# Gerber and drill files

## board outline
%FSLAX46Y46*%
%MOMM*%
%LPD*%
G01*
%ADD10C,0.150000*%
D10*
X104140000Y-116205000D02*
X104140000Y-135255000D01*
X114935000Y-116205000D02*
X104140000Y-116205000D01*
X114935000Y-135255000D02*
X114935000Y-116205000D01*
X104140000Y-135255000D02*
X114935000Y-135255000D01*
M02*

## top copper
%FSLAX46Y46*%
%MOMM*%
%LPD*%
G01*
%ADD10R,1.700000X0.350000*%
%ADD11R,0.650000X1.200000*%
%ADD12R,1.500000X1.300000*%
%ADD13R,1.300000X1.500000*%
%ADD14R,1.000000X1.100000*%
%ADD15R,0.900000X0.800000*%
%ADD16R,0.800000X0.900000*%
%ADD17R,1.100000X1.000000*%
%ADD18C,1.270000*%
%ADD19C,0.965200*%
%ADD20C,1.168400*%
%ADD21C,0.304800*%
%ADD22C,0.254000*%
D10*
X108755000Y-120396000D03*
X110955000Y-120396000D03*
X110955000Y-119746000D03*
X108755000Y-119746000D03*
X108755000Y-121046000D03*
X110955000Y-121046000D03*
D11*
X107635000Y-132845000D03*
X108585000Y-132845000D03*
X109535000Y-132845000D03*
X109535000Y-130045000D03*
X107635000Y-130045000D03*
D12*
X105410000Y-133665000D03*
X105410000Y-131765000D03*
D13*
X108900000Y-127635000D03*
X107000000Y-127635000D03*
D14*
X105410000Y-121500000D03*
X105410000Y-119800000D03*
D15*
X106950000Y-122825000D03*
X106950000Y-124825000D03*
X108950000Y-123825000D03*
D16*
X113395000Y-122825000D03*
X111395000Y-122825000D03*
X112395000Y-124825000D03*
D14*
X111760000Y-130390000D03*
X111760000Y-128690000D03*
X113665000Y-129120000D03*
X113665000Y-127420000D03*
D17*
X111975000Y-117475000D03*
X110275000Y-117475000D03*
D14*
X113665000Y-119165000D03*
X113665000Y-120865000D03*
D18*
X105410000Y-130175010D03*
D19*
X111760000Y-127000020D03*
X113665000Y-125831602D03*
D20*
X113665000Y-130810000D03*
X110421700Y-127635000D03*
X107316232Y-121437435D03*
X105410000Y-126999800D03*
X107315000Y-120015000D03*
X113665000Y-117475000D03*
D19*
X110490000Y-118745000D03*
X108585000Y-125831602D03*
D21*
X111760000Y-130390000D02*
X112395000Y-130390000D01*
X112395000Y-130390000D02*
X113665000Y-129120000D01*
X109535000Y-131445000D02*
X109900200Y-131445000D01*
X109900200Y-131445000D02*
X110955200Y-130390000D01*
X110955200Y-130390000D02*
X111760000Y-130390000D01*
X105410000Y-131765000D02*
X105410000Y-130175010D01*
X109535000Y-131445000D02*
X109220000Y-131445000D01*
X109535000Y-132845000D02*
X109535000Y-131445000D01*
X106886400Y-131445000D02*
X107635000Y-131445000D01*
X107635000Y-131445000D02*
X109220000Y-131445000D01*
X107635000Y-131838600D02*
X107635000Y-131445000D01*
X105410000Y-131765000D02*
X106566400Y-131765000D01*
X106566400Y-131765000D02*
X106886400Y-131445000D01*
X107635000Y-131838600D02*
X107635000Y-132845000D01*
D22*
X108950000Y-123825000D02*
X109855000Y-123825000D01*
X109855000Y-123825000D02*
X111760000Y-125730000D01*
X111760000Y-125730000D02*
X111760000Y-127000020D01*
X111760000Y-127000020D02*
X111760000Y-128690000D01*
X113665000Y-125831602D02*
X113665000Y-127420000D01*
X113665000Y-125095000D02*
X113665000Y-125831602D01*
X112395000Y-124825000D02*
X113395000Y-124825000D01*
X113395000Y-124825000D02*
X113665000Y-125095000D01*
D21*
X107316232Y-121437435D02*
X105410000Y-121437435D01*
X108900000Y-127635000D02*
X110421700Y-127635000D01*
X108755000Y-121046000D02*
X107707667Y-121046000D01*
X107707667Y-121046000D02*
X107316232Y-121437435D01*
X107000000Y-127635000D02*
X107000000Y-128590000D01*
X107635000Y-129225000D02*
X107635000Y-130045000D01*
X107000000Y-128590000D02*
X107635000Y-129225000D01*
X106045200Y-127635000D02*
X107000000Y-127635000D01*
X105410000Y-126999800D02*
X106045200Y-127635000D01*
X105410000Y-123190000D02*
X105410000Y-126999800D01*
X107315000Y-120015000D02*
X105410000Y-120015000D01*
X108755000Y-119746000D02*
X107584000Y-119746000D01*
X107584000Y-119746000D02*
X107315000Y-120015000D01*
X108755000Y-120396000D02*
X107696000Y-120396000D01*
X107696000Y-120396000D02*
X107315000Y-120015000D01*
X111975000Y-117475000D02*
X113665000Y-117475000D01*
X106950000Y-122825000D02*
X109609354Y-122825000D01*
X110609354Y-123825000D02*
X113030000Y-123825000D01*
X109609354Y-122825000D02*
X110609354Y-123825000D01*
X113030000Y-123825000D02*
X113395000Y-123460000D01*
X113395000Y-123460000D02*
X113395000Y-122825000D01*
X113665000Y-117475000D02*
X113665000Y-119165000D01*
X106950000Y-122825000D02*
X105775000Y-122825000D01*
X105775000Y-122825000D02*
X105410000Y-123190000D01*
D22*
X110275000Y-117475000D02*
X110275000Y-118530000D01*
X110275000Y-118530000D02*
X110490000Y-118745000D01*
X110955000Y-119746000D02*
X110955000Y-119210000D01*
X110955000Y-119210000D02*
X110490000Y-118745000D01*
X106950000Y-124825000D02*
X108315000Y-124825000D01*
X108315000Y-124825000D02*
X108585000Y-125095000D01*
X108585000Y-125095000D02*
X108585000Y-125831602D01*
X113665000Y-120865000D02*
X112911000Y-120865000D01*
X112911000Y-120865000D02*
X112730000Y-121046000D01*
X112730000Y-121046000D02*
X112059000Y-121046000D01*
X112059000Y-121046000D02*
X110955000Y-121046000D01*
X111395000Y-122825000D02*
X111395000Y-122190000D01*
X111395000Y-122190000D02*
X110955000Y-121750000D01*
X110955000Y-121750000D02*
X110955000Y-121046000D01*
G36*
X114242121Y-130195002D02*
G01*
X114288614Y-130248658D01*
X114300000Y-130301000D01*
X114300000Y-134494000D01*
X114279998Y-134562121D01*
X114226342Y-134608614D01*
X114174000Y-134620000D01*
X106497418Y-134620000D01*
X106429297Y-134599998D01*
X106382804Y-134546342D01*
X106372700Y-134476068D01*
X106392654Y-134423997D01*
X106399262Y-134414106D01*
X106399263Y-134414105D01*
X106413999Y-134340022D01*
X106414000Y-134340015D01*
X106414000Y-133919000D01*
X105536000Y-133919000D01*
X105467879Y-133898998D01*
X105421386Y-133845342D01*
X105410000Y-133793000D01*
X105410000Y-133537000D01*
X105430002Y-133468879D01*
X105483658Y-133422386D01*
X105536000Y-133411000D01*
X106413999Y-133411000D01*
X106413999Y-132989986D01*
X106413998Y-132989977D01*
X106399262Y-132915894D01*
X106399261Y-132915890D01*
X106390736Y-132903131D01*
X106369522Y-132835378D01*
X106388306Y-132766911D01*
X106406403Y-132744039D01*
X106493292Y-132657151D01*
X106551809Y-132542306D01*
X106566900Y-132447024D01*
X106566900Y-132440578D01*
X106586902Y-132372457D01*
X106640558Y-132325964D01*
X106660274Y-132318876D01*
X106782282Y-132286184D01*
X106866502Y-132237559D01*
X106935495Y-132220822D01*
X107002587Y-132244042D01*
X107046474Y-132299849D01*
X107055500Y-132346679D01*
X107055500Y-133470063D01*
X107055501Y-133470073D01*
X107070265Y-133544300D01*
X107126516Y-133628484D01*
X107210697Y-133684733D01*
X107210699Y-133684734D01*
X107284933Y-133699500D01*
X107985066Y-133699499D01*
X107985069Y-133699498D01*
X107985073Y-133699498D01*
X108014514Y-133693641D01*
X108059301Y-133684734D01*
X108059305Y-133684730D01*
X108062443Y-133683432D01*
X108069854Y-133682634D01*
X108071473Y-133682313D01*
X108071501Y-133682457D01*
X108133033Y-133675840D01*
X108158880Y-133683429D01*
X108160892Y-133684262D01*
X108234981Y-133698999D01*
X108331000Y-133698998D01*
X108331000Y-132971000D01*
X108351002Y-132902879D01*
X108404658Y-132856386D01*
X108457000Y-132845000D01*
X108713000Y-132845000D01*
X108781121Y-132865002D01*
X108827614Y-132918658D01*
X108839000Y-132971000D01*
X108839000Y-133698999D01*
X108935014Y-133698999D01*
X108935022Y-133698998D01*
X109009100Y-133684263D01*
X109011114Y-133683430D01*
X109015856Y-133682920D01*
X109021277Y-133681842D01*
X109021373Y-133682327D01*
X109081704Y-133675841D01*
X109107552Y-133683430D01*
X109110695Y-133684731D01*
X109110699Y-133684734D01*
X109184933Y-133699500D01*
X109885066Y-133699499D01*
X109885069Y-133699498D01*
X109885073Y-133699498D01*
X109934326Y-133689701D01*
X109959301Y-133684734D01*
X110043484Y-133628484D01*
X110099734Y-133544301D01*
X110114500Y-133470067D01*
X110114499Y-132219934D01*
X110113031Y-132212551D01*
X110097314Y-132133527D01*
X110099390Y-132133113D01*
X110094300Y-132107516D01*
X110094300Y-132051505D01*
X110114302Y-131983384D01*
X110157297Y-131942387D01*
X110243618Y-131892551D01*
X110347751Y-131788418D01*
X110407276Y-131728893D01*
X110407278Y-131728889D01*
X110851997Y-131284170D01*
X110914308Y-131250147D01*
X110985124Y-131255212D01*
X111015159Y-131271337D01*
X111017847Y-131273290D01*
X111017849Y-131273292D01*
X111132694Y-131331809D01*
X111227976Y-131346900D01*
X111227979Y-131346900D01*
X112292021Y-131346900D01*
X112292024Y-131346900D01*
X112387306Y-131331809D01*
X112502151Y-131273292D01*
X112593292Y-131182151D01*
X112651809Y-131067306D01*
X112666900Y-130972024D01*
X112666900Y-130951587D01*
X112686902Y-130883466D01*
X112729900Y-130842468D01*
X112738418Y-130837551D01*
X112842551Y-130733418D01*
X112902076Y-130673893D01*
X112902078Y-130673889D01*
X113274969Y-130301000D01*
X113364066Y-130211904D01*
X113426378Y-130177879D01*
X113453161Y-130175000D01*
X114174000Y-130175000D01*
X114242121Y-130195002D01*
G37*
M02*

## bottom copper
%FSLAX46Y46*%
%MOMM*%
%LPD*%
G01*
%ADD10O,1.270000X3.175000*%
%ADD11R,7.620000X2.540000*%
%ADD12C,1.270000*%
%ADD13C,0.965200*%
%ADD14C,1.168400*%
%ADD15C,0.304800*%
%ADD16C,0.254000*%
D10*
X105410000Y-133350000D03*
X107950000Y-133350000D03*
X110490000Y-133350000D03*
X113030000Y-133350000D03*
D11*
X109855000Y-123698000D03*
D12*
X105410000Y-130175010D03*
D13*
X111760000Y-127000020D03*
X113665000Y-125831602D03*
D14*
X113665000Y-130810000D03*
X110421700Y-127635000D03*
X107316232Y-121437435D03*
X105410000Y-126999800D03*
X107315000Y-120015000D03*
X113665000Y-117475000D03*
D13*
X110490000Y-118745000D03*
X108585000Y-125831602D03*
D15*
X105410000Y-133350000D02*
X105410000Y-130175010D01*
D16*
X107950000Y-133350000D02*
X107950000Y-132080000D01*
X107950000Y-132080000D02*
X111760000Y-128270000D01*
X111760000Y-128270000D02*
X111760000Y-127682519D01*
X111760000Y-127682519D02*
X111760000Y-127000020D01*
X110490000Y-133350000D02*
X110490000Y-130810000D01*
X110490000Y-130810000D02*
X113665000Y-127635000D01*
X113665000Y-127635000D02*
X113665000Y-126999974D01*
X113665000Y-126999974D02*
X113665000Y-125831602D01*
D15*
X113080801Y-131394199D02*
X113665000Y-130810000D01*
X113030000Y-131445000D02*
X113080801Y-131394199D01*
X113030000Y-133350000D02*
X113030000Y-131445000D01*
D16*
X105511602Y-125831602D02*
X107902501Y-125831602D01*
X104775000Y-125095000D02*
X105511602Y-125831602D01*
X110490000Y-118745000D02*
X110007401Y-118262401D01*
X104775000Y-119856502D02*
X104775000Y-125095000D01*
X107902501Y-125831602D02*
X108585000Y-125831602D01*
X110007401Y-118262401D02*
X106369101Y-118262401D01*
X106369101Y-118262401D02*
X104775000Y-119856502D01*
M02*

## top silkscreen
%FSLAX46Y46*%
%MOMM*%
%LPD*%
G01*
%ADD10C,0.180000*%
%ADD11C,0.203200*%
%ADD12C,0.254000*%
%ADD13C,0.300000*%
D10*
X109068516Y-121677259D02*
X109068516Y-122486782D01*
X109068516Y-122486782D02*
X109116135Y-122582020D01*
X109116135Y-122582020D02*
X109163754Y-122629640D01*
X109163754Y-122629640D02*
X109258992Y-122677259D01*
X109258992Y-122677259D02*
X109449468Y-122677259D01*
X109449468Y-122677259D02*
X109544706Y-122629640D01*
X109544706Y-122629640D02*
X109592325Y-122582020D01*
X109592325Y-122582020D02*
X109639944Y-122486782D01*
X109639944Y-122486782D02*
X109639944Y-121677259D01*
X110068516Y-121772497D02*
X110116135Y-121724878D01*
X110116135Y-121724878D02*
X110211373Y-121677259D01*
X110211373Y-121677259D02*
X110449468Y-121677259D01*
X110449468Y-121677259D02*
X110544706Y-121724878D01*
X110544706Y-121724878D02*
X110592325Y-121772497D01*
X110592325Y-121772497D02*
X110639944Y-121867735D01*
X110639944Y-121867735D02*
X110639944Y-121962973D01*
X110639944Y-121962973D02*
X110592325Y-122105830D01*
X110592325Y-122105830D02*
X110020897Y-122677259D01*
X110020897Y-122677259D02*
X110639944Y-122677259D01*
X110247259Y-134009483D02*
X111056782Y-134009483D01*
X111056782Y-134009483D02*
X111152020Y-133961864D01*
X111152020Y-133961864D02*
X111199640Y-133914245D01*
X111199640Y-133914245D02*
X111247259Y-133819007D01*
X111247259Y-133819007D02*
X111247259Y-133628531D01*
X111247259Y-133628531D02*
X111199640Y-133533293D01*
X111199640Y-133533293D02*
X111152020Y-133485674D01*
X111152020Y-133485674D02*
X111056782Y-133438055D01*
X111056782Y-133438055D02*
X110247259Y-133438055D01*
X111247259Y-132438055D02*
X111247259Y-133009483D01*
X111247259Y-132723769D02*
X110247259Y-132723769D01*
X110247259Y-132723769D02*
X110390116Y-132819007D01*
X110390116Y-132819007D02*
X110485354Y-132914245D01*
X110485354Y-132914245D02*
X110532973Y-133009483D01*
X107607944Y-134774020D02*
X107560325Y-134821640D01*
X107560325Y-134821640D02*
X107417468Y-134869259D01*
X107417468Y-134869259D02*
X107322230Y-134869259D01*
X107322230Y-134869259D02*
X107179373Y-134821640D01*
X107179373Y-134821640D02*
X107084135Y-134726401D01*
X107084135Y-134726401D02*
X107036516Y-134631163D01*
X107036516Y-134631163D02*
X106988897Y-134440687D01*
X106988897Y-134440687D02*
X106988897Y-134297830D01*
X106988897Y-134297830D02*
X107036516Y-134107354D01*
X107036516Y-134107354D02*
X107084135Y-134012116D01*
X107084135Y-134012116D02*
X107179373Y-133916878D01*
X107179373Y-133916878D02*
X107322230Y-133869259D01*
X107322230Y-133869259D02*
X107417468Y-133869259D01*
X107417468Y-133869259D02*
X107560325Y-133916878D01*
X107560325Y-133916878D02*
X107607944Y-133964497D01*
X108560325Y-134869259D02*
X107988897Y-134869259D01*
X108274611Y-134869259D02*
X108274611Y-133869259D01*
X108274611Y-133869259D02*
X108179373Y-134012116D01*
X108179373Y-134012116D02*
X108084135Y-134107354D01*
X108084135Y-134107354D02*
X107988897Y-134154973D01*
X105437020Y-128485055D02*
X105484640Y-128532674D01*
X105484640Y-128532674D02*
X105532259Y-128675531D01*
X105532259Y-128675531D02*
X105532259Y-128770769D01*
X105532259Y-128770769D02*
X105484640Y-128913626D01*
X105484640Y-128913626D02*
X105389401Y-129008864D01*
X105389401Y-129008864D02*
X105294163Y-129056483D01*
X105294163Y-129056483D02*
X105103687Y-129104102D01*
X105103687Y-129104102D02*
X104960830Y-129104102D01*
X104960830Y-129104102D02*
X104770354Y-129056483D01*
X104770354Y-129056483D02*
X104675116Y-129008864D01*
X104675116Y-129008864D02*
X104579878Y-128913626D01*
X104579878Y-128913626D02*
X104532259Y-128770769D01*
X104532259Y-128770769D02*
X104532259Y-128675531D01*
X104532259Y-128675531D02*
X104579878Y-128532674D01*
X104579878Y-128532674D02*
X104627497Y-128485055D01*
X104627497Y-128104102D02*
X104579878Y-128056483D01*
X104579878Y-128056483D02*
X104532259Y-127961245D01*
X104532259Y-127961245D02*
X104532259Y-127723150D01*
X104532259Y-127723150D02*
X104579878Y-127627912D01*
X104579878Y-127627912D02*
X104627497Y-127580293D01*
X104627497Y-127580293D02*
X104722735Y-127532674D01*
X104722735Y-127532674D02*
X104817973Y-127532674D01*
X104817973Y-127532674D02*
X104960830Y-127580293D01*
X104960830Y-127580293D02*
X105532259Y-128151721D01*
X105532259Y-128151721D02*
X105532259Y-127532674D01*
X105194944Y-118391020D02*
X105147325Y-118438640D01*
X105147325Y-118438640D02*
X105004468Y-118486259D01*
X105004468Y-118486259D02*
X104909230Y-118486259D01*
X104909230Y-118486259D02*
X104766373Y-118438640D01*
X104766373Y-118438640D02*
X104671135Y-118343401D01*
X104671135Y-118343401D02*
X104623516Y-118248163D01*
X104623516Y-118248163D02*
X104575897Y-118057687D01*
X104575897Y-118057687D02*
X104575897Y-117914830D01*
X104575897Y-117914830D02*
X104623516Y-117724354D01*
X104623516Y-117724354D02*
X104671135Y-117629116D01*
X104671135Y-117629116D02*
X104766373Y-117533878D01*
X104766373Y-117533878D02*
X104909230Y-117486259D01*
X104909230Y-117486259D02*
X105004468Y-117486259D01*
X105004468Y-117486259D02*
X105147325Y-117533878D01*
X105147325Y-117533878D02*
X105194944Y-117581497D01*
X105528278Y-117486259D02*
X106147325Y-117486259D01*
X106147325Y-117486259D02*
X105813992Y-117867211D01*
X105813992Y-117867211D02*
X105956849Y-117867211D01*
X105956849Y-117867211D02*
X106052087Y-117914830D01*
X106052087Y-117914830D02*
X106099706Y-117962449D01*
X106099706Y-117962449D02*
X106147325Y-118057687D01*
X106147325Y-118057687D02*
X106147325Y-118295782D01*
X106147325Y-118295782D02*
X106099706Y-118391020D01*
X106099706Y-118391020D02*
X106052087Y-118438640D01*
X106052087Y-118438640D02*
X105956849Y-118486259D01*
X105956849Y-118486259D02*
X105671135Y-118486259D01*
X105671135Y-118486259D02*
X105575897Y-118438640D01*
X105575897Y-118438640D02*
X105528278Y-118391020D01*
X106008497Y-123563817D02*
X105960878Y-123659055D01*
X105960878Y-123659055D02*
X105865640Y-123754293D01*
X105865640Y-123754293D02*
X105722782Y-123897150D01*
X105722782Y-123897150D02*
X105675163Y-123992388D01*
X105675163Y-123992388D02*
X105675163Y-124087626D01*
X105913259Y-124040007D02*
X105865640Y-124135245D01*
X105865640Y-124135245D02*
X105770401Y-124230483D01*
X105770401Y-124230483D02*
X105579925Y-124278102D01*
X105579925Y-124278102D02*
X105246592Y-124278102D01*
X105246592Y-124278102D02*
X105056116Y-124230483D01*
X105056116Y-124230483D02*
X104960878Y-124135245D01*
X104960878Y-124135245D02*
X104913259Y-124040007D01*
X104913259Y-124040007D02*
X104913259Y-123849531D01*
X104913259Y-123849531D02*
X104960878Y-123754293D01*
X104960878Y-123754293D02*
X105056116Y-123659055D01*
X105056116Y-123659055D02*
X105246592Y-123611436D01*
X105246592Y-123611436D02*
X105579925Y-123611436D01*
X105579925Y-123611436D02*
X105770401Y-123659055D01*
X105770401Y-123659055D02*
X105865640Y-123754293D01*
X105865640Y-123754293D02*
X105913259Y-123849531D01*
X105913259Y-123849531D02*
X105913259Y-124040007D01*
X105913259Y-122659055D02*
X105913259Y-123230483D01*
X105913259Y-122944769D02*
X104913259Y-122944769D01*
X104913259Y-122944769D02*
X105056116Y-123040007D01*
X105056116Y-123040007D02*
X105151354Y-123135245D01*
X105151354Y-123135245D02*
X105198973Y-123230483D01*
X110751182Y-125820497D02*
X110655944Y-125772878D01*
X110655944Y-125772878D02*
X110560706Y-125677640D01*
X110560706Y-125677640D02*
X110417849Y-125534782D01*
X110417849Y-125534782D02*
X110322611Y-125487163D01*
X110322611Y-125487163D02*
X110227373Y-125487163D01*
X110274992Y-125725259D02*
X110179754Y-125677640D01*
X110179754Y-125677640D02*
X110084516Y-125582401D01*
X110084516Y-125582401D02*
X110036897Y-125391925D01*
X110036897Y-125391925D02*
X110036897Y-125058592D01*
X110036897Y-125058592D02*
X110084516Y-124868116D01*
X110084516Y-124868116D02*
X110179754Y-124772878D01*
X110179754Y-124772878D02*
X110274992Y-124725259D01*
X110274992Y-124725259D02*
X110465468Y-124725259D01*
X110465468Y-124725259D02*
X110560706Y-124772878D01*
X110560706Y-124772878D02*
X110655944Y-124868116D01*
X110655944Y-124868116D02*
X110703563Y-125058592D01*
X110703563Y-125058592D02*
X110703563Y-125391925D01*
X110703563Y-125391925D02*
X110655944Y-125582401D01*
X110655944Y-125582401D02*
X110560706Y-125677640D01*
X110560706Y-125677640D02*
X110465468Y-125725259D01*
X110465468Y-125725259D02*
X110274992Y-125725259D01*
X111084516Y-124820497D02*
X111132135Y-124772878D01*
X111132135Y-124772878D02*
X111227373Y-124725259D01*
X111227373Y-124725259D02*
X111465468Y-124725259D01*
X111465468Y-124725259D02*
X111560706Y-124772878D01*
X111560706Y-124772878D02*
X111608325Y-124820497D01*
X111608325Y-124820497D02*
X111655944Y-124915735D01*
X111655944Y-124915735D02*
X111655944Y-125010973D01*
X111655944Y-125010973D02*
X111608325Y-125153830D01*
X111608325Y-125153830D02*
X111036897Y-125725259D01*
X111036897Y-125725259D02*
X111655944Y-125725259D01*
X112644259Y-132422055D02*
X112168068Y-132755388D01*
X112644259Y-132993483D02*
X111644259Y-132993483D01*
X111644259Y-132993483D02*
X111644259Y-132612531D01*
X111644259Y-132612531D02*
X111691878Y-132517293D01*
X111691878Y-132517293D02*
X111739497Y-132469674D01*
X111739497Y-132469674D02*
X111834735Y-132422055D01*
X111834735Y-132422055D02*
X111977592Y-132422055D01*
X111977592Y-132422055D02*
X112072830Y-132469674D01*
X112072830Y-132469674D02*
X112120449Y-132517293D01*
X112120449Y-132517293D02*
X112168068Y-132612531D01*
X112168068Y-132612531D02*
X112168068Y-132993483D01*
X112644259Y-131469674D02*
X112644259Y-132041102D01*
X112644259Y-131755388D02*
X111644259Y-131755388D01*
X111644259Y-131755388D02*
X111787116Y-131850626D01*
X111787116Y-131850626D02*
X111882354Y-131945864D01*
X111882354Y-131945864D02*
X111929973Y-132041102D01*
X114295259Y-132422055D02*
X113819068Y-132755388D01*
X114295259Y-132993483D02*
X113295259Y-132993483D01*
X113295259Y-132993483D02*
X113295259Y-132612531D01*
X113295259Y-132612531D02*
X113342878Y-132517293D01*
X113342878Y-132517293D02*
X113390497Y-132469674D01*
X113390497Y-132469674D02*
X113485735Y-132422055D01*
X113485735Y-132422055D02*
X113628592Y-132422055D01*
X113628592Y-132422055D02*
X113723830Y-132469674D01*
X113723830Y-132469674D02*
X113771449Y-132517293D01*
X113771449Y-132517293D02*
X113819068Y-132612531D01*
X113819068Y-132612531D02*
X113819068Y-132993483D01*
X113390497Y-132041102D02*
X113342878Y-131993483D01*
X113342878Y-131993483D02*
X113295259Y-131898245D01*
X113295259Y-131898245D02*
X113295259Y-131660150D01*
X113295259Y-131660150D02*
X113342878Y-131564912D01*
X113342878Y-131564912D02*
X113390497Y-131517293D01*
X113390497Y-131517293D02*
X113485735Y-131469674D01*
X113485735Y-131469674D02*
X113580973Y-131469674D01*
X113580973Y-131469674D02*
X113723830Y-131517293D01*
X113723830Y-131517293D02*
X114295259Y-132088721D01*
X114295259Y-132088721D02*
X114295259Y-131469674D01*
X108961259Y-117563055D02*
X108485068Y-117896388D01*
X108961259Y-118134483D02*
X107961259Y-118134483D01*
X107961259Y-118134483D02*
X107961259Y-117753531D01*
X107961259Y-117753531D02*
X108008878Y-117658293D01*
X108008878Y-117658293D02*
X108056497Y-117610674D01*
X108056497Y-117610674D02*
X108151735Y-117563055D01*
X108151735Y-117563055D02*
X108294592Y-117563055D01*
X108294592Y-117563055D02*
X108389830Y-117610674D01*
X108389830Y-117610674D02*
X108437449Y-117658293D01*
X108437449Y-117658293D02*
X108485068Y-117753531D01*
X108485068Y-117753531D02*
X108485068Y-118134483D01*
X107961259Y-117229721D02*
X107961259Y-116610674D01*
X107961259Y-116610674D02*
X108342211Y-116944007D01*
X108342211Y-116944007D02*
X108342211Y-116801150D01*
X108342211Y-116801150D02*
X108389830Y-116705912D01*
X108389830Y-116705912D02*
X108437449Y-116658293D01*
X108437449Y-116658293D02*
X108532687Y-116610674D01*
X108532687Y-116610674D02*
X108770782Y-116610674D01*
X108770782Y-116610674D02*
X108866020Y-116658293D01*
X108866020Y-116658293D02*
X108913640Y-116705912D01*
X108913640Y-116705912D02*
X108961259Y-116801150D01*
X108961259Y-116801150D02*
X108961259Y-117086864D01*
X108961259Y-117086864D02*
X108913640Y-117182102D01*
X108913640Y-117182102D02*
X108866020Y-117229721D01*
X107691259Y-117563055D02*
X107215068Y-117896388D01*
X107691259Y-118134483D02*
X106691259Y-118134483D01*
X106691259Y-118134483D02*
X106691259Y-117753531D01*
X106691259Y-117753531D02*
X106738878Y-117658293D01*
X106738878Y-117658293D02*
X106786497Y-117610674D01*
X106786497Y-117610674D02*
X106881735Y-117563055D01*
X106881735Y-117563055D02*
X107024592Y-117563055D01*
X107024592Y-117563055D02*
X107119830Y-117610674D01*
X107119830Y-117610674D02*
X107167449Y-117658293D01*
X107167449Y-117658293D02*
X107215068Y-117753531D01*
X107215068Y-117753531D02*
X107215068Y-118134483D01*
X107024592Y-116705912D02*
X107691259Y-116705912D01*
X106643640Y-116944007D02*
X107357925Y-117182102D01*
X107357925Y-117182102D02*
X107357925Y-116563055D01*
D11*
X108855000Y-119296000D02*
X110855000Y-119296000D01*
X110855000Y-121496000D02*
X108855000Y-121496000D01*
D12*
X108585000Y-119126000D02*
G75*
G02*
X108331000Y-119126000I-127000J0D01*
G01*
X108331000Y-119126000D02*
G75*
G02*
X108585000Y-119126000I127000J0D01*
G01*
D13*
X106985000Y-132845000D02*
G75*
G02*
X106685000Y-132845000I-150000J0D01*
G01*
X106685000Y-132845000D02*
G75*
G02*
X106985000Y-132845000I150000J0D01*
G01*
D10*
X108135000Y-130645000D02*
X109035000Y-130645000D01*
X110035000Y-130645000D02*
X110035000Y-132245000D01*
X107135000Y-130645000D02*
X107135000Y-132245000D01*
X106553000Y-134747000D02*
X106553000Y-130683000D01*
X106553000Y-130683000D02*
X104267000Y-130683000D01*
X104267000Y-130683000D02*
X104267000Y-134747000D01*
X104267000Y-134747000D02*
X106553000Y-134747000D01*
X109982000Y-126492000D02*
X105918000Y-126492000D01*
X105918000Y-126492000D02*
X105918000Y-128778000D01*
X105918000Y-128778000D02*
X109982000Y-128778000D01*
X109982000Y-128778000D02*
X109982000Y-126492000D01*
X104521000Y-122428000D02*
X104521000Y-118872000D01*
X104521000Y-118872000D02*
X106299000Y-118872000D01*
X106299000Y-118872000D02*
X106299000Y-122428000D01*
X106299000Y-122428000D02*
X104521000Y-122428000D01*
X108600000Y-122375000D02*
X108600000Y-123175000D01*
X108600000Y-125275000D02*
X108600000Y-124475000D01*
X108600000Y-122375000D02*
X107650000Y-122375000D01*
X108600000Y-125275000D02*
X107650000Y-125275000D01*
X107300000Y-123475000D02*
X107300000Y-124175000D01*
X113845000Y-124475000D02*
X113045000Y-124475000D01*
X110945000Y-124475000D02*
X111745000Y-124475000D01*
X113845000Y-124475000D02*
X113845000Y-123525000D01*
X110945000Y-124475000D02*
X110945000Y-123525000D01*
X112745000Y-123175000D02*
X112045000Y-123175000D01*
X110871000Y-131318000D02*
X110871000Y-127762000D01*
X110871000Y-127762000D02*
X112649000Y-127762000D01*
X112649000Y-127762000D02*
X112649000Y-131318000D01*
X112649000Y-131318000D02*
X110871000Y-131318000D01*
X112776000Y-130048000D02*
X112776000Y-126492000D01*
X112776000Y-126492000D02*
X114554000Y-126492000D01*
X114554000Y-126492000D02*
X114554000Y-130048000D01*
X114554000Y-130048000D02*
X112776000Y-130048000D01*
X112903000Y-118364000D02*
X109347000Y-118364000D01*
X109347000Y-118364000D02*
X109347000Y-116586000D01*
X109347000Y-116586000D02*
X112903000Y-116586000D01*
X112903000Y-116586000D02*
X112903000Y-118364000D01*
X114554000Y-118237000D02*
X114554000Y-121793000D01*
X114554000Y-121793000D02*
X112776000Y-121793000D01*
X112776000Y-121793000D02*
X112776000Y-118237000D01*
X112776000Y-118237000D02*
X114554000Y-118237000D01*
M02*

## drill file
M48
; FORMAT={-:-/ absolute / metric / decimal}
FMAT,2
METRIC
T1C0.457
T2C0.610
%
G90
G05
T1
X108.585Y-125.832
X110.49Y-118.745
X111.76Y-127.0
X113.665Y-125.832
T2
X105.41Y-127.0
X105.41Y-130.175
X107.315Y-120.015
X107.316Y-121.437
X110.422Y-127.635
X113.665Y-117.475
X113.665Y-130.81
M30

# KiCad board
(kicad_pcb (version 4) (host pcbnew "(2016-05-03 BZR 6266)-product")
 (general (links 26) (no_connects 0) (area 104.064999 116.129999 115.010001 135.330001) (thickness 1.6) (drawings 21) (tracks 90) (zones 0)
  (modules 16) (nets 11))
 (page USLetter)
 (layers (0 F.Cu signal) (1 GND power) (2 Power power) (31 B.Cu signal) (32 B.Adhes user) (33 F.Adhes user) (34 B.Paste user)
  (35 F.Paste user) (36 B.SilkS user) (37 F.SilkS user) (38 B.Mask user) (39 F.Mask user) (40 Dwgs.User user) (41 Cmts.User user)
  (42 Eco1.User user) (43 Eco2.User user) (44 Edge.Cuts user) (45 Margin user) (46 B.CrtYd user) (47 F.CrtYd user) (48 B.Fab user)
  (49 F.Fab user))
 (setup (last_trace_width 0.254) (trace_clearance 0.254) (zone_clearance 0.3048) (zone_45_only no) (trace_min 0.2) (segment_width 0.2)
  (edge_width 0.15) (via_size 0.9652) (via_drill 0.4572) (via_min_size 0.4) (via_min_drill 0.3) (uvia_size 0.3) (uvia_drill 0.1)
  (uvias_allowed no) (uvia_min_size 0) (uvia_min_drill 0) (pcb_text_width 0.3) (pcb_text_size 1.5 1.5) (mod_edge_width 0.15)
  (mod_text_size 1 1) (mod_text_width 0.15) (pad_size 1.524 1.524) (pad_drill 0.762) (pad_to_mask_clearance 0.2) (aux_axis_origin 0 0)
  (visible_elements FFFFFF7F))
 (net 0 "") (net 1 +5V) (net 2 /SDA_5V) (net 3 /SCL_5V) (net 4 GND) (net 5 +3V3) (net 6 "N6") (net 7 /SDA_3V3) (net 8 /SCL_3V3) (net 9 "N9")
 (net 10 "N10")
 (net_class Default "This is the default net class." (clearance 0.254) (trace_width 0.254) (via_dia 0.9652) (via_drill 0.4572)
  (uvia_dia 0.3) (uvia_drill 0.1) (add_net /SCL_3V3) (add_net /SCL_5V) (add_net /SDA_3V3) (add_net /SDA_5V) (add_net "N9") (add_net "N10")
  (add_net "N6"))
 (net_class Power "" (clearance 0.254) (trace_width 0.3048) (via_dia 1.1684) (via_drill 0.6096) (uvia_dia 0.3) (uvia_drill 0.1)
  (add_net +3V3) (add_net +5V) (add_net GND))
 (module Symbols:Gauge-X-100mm (layer B.Cu) (at 97.79 135.255 90)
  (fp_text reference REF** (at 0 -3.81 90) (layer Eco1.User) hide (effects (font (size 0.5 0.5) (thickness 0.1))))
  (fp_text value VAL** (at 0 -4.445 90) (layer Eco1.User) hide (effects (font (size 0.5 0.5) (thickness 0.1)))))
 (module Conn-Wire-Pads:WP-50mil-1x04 (layer B.Cu) (at 109.22 133.35)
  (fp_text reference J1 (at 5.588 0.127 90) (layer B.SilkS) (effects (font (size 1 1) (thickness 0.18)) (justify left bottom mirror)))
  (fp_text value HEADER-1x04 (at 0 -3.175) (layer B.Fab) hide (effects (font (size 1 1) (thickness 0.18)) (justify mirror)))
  (pad 1 smd oval (at -3.81 0) (size 1.27 3.175) (layers B.Cu B.Paste B.Mask) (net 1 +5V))
  (pad 2 smd oval (at -1.27 0) (size 1.27 3.175) (layers B.Cu B.Paste B.Mask) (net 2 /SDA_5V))
  (pad 3 smd oval (at 1.27 0) (size 1.27 3.175) (layers B.Cu B.Paste B.Mask) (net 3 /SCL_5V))
  (pad 4 smd oval (at 3.81 0) (size 1.27 3.175) (layers B.Cu B.Paste B.Mask) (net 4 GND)))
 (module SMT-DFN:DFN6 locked (layer F.Cu) (at 109.855 120.396)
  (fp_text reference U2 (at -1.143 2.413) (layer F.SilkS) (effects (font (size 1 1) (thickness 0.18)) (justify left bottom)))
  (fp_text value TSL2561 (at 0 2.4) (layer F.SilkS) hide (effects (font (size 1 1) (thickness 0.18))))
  (fp_line (start -1 -1.1) (end 1 -1.1) (layer F.SilkS) (width 0.2032))
  (fp_line (start 1 1.1) (end -1 1.1) (layer F.SilkS) (width 0.2032))
  (fp_circle (center -1.397 -1.27) (end -1.27 -1.27) (layer F.SilkS) (width 0.254))
  (pad 2 smd rect (at -1.1 0) (size 1.7 0.35) (layers F.Cu F.Paste F.Mask) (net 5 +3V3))
  (pad 5 smd rect (at 1.1 0) (size 1.7 0.35) (layers F.Cu F.Paste F.Mask) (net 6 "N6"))
  (pad 6 smd rect (at 1.1 -0.65) (size 1.7 0.35) (layers F.Cu F.Paste F.Mask) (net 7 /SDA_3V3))
  (pad 1 smd rect (at -1.1 -0.65) (size 1.7 0.35) (layers F.Cu F.Paste F.Mask) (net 5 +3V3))
  (pad 3 smd rect (at -1.1 0.65) (size 1.7 0.35) (layers F.Cu F.Paste F.Mask) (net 4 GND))
  (pad 4 smd rect (at 1.1 0.65) (size 1.7 0.35) (layers F.Cu F.Paste F.Mask) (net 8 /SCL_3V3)))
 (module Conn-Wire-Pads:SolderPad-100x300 (layer B.Cu) (at 109.855 123.698)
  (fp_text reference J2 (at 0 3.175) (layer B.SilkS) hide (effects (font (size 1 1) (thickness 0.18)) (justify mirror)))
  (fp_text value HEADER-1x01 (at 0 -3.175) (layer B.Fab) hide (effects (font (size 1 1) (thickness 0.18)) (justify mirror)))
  (pad 1 smd rect (at 0 0) (size 7.62 2.54) (layers B.Cu B.Paste B.Mask) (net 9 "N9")))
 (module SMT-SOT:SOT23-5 (layer F.Cu) (at 108.585 131.445) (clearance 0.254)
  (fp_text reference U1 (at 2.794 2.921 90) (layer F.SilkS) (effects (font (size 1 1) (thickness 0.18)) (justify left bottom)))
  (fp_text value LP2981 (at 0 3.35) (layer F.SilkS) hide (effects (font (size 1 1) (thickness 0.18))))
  (fp_circle (center -1.75 1.4) (end -1.6 1.4) (layer F.SilkS) (width 0.3))
  (fp_line (start -0.45 -0.8) (end 0.45 -0.8) (layer F.SilkS) (width 0.18))
  (fp_line (start 1.45 -0.8) (end 1.45 0.8) (layer F.SilkS) (width 0.18))
  (fp_line (start -1.45 -0.8) (end -1.45 0.8) (layer F.SilkS) (width 0.18))
  (pad 1 smd rect (at -0.95 1.4) (size 0.65 1.2) (layers F.Cu F.Paste F.Mask) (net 1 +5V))
  (pad 2 smd rect (at 0 1.4) (size 0.65 1.2) (layers F.Cu F.Paste F.Mask) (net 4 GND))
  (pad 3 smd rect (at 0.95 1.4) (size 0.65 1.2) (layers F.Cu F.Paste F.Mask) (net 1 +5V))
  (pad 4 smd rect (at 0.95 -1.4) (size 0.65 1.2) (layers F.Cu F.Paste F.Mask) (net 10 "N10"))
  (pad 5 smd rect (at -0.95 -1.4) (size 0.65 1.2) (layers F.Cu F.Paste F.Mask) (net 5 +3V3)))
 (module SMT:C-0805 (layer F.Cu) (at 105.41 132.715 90)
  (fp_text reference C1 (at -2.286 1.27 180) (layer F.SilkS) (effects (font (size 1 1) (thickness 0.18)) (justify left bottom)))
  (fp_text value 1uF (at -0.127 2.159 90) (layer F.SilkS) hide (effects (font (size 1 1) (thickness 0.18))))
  (fp_line (start -2.032 1.143) (end 2.032 1.143) (layer F.SilkS) (width 0.18))
  (fp_line (start 2.032 1.143) (end 2.032 -1.143) (layer F.SilkS) (width 0.18))
  (fp_line (start 2.032 -1.143) (end -2.032 -1.143) (layer F.SilkS) (width 0.18))
  (fp_line (start -2.032 -1.143) (end -2.032 1.143) (layer F.SilkS) (width 0.18))
  (pad 1 smd rect (at -0.95 0 90) (size 1.3 1.5) (layers F.Cu F.Paste F.Mask) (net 4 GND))
  (pad 2 smd rect (at 0.95 0 90) (size 1.3 1.5) (layers F.Cu F.Paste F.Mask) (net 1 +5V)))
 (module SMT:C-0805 (layer F.Cu) (at 107.95 127.635 180)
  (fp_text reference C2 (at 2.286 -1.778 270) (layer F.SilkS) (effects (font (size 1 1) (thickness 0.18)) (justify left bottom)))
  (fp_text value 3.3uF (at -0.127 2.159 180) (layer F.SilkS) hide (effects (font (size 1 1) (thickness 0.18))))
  (fp_line (start -2.032 1.143) (end 2.032 1.143) (layer F.SilkS) (width 0.18))
  (fp_line (start 2.032 1.143) (end 2.032 -1.143) (layer F.SilkS) (width 0.18))
  (fp_line (start 2.032 -1.143) (end -2.032 -1.143) (layer F.SilkS) (width 0.18))
  (fp_line (start -2.032 -1.143) (end -2.032 1.143) (layer F.SilkS) (width 0.18))
  (pad 1 smd rect (at -0.95 0 180) (size 1.3 1.5) (layers F.Cu F.Paste F.Mask) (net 4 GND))
  (pad 2 smd rect (at 0.95 0 180) (size 1.3 1.5) (layers F.Cu F.Paste F.Mask) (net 5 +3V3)))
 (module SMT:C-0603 (layer F.Cu) (at 105.41 120.65 90)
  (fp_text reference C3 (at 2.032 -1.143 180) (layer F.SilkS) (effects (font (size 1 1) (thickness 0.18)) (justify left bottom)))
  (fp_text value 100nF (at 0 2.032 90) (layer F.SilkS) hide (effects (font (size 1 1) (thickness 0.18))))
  (fp_line (start -1.778 -0.889) (end 1.778 -0.889) (layer F.SilkS) (width 0.18))
  (fp_line (start 1.778 -0.889) (end 1.778 0.889) (layer F.SilkS) (width 0.18))
  (fp_line (start 1.778 0.889) (end -1.778 0.889) (layer F.SilkS) (width 0.18))
  (fp_line (start -1.778 0.889) (end -1.778 -0.889) (layer F.SilkS) (width 0.18))
  (pad 1 smd rect (at -0.85 0 90) (size 1.1 1) (layers F.Cu F.Paste F.Mask) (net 4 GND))
  (pad 2 smd rect (at 0.85 0 90) (size 1.1 1) (layers F.Cu F.Paste F.Mask) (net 5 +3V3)))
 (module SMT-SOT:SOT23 (layer F.Cu) (at 107.95 123.825 270)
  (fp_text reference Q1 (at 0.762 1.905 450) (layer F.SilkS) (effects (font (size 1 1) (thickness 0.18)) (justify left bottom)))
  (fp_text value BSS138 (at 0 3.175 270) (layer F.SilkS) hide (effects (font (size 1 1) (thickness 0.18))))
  (fp_line (start -1.45 -0.65) (end -0.65 -0.65) (layer F.SilkS) (width 0.18))
  (fp_line (start 1.45 -0.65) (end 0.65 -0.65) (layer F.SilkS) (width 0.18))
  (fp_line (start -1.45 -0.65) (end -1.45 0.3) (layer F.SilkS) (width 0.18))
  (fp_line (start 1.45 -0.65) (end 1.45 0.3) (layer F.SilkS) (width 0.18))
  (fp_line (start -0.35 0.65) (end 0.35 0.65) (layer F.SilkS) (width 0.18))
  (pad 1 smd rect (at -1 1 270) (size 0.8 0.9) (layers F.Cu F.Paste F.Mask) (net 5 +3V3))
  (pad 2 smd rect (at 1 1 270) (size 0.8 0.9) (layers F.Cu F.Paste F.Mask) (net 7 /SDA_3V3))
  (pad 3 smd rect (at 0 -1 270) (size 0.8 0.9) (layers F.Cu F.Paste F.Mask) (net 2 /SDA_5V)))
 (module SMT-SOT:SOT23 (layer F.Cu) (at 112.395 123.825 180)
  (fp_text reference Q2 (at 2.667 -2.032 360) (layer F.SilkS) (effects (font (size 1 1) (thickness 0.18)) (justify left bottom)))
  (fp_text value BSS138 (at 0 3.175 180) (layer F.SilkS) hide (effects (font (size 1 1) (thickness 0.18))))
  (fp_line (start -1.45 -0.65) (end -0.65 -0.65) (layer F.SilkS) (width 0.18))
  (fp_line (start 1.45 -0.65) (end 0.65 -0.65) (layer F.SilkS) (width 0.18))
  (fp_line (start -1.45 -0.65) (end -1.45 0.3) (layer F.SilkS) (width 0.18))
  (fp_line (start 1.45 -0.65) (end 1.45 0.3) (layer F.SilkS) (width 0.18))
  (fp_line (start -0.35 0.65) (end 0.35 0.65) (layer F.SilkS) (width 0.18))
  (pad 1 smd rect (at -1 1 180) (size 0.8 0.9) (layers F.Cu F.Paste F.Mask) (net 5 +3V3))
  (pad 2 smd rect (at 1 1 180) (size 0.8 0.9) (layers F.Cu F.Paste F.Mask) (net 8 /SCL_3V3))
  (pad 3 smd rect (at 0 -1 180) (size 0.8 0.9) (layers F.Cu F.Paste F.Mask) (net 3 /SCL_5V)))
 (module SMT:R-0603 (layer F.Cu) (at 111.76 129.54 90)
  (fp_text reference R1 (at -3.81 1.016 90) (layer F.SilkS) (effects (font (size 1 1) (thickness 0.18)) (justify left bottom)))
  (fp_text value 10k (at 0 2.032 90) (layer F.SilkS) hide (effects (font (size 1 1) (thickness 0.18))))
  (fp_line (start -1.778 -0.889) (end 1.778 -0.889) (layer F.SilkS) (width 0.18))
  (fp_line (start 1.778 -0.889) (end 1.778 0.889) (layer F.SilkS) (width 0.18))
  (fp_line (start 1.778 0.889) (end -1.778 0.889) (layer F.SilkS) (width 0.18))
  (fp_line (start -1.778 0.889) (end -1.778 -0.889) (layer F.SilkS) (width 0.18))
  (pad 1 smd rect (at -0.85 0 90) (size 1.1 1) (layers F.Cu F.Paste F.Mask) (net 1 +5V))
  (pad 2 smd rect (at 0.85 0 90) (size 1.1 1) (layers F.Cu F.Paste F.Mask) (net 2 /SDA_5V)))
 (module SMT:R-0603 (layer F.Cu) (at 113.665 128.27 90)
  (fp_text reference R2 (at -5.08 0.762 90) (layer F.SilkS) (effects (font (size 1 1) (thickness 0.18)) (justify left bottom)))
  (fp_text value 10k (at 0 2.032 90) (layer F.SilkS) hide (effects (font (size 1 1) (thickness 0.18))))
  (fp_line (start -1.778 -0.889) (end 1.778 -0.889) (layer F.SilkS) (width 0.18))
  (fp_line (start 1.778 -0.889) (end 1.778 0.889) (layer F.SilkS) (width 0.18))
  (fp_line (start 1.778 0.889) (end -1.778 0.889) (layer F.SilkS) (width 0.18))
  (fp_line (start -1.778 0.889) (end -1.778 -0.889) (layer F.SilkS) (width 0.18))
  (pad 1 smd rect (at -0.85 0 90) (size 1.1 1) (layers F.Cu F.Paste F.Mask) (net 1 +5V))
  (pad 2 smd rect (at 0.85 0 90) (size 1.1 1) (layers F.Cu F.Paste F.Mask) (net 3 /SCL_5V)))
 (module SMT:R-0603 (layer F.Cu) (at 111.125 117.475 180)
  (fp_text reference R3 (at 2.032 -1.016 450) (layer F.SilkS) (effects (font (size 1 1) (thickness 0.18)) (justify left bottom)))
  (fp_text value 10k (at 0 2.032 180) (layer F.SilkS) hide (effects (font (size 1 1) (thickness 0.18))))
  (fp_line (start -1.778 -0.889) (end 1.778 -0.889) (layer F.SilkS) (width 0.18))
  (fp_line (start 1.778 -0.889) (end 1.778 0.889) (layer F.SilkS) (width 0.18))
  (fp_line (start 1.778 0.889) (end -1.778 0.889) (layer F.SilkS) (width 0.18))
  (fp_line (start -1.778 0.889) (end -1.778 -0.889) (layer F.SilkS) (width 0.18))
  (pad 1 smd rect (at -0.85 0 180) (size 1.1 1) (layers F.Cu F.Paste F.Mask) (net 5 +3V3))
  (pad 2 smd rect (at 0.85 0 180) (size 1.1 1) (layers F.Cu F.Paste F.Mask) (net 7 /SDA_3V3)))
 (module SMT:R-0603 (layer F.Cu) (at 113.665 120.015 270)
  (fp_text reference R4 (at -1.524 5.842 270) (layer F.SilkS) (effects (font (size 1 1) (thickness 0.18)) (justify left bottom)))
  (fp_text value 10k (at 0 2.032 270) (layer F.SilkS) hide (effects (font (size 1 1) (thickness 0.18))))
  (fp_line (start -1.778 -0.889) (end 1.778 -0.889) (layer F.SilkS) (width 0.18))
  (fp_line (start 1.778 -0.889) (end 1.778 0.889) (layer F.SilkS) (width 0.18))
  (fp_line (start 1.778 0.889) (end -1.778 0.889) (layer F.SilkS) (width 0.18))
  (fp_line (start -1.778 0.889) (end -1.778 -0.889) (layer F.SilkS) (width 0.18))
  (pad 1 smd rect (at -0.85 0 270) (size 1.1 1) (layers F.Cu F.Paste F.Mask) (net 5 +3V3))
  (pad 2 smd rect (at 0.85 0 270) (size 1.1 1) (layers F.Cu F.Paste F.Mask) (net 8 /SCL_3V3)))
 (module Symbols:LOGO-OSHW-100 (layer B.Cu) (at 106.172 117.983 180)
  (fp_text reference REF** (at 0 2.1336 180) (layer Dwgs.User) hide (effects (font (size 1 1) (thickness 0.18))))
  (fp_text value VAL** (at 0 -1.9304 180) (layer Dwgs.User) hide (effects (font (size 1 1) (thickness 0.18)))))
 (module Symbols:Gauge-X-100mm (layer F.Cu) (at 104.14 141.605)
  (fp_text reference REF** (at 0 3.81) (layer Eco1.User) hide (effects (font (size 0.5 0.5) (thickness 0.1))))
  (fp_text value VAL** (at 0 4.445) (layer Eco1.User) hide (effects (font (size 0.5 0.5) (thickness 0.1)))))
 (gr_line (start 104.14 116.205) (end 104.14 135.255) (layer Edge.Cuts) (width 0.15))
 (gr_line (start 114.935 116.205) (end 104.14 116.205) (layer Edge.Cuts) (width 0.15))
 (gr_line (start 114.935 135.255) (end 114.935 116.205) (layer Edge.Cuts) (width 0.15))
 (gr_line (start 104.14 135.255) (end 114.935 135.255) (layer Edge.Cuts) (width 0.15))
 (segment (start 111.76 130.39) (end 112.395 130.39) (width 0.3048) (layer F.Cu) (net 1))
 (segment (start 112.395 130.39) (end 113.665 129.12) (width 0.3048) (layer F.Cu) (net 1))
 (segment (start 109.535 131.445) (end 109.9002 131.445) (width 0.3048) (layer F.Cu) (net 1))
 (segment (start 109.9002 131.445) (end 110.9552 130.39) (width 0.3048) (layer F.Cu) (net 1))
 (segment (start 110.9552 130.39) (end 111.76 130.39) (width 0.3048) (layer F.Cu) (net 1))
 (via (at 105.41 130.17501) (size 1.27) (drill 0.6096) (layers F.Cu B.Cu) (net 1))
 (segment (start 105.41 131.765) (end 105.41 130.17501) (width 0.3048) (layer F.Cu) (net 1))
 (segment (start 109.535 131.445) (end 109.22 131.445) (width 0.3048) (layer F.Cu) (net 1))
 (segment (start 109.535 132.845) (end 109.535 131.445) (width 0.3048) (layer F.Cu) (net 1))
 (segment (start 106.8864 131.445) (end 107.635 131.445) (width 0.3048) (layer F.Cu) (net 1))
 (segment (start 107.635 131.445) (end 109.22 131.445) (width 0.3048) (layer F.Cu) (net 1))
 (segment (start 107.635 131.8386) (end 107.635 131.445) (width 0.3048) (layer F.Cu) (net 1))
 (segment (start 105.41 131.765) (end 106.5664 131.765) (width 0.3048) (layer F.Cu) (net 1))
 (segment (start 106.5664 131.765) (end 106.8864 131.445) (width 0.3048) (layer F.Cu) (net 1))
 (segment (start 107.635 131.8386) (end 107.635 132.845) (width 0.3048) (layer F.Cu) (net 1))
 (segment (start 105.41 133.35) (end 105.41 130.17501) (width 0.3048) (layer B.Cu) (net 1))
 (segment (start 107.95 133.35) (end 107.95 132.08) (width 0.254) (layer B.Cu) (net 2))
 (segment (start 107.95 132.08) (end 111.76 128.27) (width 0.254) (layer B.Cu) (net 2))
 (segment (start 111.76 128.27) (end 111.76 127.682519) (width 0.254) (layer B.Cu) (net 2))
 (segment (start 111.76 127.682519) (end 111.76 127.00002) (width 0.254) (layer B.Cu) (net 2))
 (segment (start 108.95 123.825) (end 109.855 123.825) (width 0.254) (layer F.Cu) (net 2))
 (segment (start 109.855 123.825) (end 111.76 125.73) (width 0.254) (layer F.Cu) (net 2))
 (segment (start 111.76 125.73) (end 111.76 127.00002) (width 0.254) (layer F.Cu) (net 2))
 (segment (start 111.76 127.00002) (end 111.76 128.69) (width 0.254) (layer F.Cu) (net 2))
 (via (at 111.76 127.00002) (size 0.9652) (drill 0.4572) (layers F.Cu B.Cu) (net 2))
 (segment (start 113.665 125.831602) (end 113.665 127.42) (width 0.254) (layer F.Cu) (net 3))
 (segment (start 113.665 125.095) (end 113.665 125.831602) (width 0.254) (layer F.Cu) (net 3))
 (segment (start 110.49 133.35) (end 110.49 130.81) (width 0.254) (layer B.Cu) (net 3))
 (segment (start 110.49 130.81) (end 113.665 127.635) (width 0.254) (layer B.Cu) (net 3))
 (segment (start 113.665 127.635) (end 113.665 126.999974) (width 0.254) (layer B.Cu) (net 3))
 (segment (start 113.665 126.999974) (end 113.665 125.831602) (width 0.254) (layer B.Cu) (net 3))
 (via (at 113.665 125.831602) (size 0.9652) (drill 0.4572) (layers F.Cu B.Cu) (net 3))
 (segment (start 112.395 124.825) (end 113.395 124.825) (width 0.254) (layer F.Cu) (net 3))
 (segment (start 113.395 124.825) (end 113.665 125.095) (width 0.254) (layer F.Cu) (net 3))
 (segment (start 107.316232 121.437435) (end 105.41 121.437435) (width 0.3048) (layer F.Cu) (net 4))
 (segment (start 113.080801 131.394199) (end 113.665 130.81) (width 0.3048) (layer B.Cu) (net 4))
 (segment (start 113.03 131.445) (end 113.080801 131.394199) (width 0.3048) (layer B.Cu) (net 4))
 (segment (start 113.03 133.35) (end 113.03 131.445) (width 0.3048) (layer B.Cu) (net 4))
 (via (at 113.665 130.81) (size 1.1684) (drill 0.6096) (layers F.Cu B.Cu) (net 4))
 (segment (start 108.9 127.635) (end 110.4217 127.635) (width 0.3048) (layer F.Cu) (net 4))
 (via (at 110.4217 127.635) (size 1.1684) (drill 0.6096) (layers F.Cu B.Cu) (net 4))
 (segment (start 108.755 121.046) (end 107.707667 121.046) (width 0.3048) (layer F.Cu) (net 4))
 (segment (start 107.707667 121.046) (end 107.316232 121.437435) (width 0.3048) (layer F.Cu) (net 4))
 (via (at 107.316232 121.437435) (size 1.1684) (drill 0.6096) (layers F.Cu B.Cu) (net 4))
 (via (at 105.41 126.9998) (size 1.1684) (drill 0.6096) (layers F.Cu B.Cu) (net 5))
 (segment (start 107 127.635) (end 107 128.59) (width 0.3048) (layer F.Cu) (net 5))
 (segment (start 107.635 129.225) (end 107.635 130.045) (width 0.3048) (layer F.Cu) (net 5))
 (segment (start 107 128.59) (end 107.635 129.225) (width 0.3048) (layer F.Cu) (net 5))
 (segment (start 106.0452 127.635) (end 107 127.635) (width 0.3048) (layer F.Cu) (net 5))
 (segment (start 105.41 126.9998) (end 106.0452 127.635) (width 0.3048) (layer F.Cu) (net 5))
 (segment (start 105.41 123.19) (end 105.41 126.9998) (width 0.3048) (layer F.Cu) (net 5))
 (segment (start 107.315 120.015) (end 105.41 120.015) (width 0.3048) (layer F.Cu) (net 5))
 (segment (start 108.755 119.746) (end 107.584 119.746) (width 0.3048) (layer F.Cu) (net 5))
 (segment (start 107.584 119.746) (end 107.315 120.015) (width 0.3048) (layer F.Cu) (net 5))
 (segment (start 108.755 120.396) (end 107.696 120.396) (width 0.3048) (layer F.Cu) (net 5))
 (segment (start 107.696 120.396) (end 107.315 120.015) (width 0.3048) (layer F.Cu) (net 5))
 (via (at 107.315 120.015) (size 1.1684) (drill 0.6096) (layers F.Cu B.Cu) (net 5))
 (segment (start 111.975 117.475) (end 113.665 117.475) (width 0.3048) (layer F.Cu) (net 5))
 (segment (start 106.95 122.825) (end 109.609354 122.825) (width 0.3048) (layer F.Cu) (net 5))
 (segment (start 110.609354 123.825) (end 113.03 123.825) (width 0.3048) (layer F.Cu) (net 5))
 (segment (start 109.609354 122.825) (end 110.609354 123.825) (width 0.3048) (layer F.Cu) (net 5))
 (segment (start 113.03 123.825) (end 113.395 123.46) (width 0.3048) (layer F.Cu) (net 5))
 (segment (start 113.395 123.46) (end 113.395 122.825) (width 0.3048) (layer F.Cu) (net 5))
 (segment (start 113.665 117.475) (end 113.665 119.165) (width 0.3048) (layer F.Cu) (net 5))
 (via (at 113.665 117.475) (size 1.1684) (drill 0.6096) (layers F.Cu B.Cu) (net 5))
 (segment (start 106.95 122.825) (end 105.775 122.825) (width 0.3048) (layer F.Cu) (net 5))
 (segment (start 105.775 122.825) (end 105.41 123.19) (width 0.3048) (layer F.Cu) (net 5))
 (segment (start 105.511602 125.831602) (end 107.902501 125.831602) (width 0.254) (layer B.Cu) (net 7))
 (segment (start 104.775 125.095) (end 105.511602 125.831602) (width 0.254) (layer B.Cu) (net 7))
 (segment (start 110.49 118.745) (end 110.007401 118.262401) (width 0.254) (layer B.Cu) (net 7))
 (segment (start 104.775 119.856502) (end 104.775 125.095) (width 0.254) (layer B.Cu) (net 7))
 (segment (start 107.902501 125.831602) (end 108.585 125.831602) (width 0.254) (layer B.Cu) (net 7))
 (segment (start 110.007401 118.262401) (end 106.369101 118.262401) (width 0.254) (layer B.Cu) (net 7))
 (segment (start 106.369101 118.262401) (end 104.775 119.856502) (width 0.254) (layer B.Cu) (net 7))
 (segment (start 110.275 117.475) (end 110.275 118.53) (width 0.254) (layer F.Cu) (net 7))
 (segment (start 110.275 118.53) (end 110.49 118.745) (width 0.254) (layer F.Cu) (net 7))
 (segment (start 110.955 119.746) (end 110.955 119.21) (width 0.254) (layer F.Cu) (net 7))
 (segment (start 110.955 119.21) (end 110.49 118.745) (width 0.254) (layer F.Cu) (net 7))
 (via (at 110.49 118.745) (size 0.9652) (drill 0.4572) (layers F.Cu B.Cu) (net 7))
 (segment (start 106.95 124.825) (end 108.315 124.825) (width 0.254) (layer F.Cu) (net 7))
 (segment (start 108.315 124.825) (end 108.585 125.095) (width 0.254) (layer F.Cu) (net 7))
 (segment (start 108.585 125.095) (end 108.585 125.831602) (width 0.254) (layer F.Cu) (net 7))
 (via (at 108.585 125.831602) (size 0.9652) (drill 0.4572) (layers F.Cu B.Cu) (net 7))
 (segment (start 113.665 120.865) (end 112.911 120.865) (width 0.254) (layer F.Cu) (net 8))
 (segment (start 112.911 120.865) (end 112.73 121.046) (width 0.254) (layer F.Cu) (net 8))
 (segment (start 112.73 121.046) (end 112.059 121.046) (width 0.254) (layer F.Cu) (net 8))
 (segment (start 112.059 121.046) (end 110.955 121.046) (width 0.254) (layer F.Cu) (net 8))
 (segment (start 111.395 122.825) (end 111.395 122.19) (width 0.254) (layer F.Cu) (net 8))
 (segment (start 111.395 122.19) (end 110.955 121.75) (width 0.254) (layer F.Cu) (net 8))
 (segment (start 110.955 121.75) (end 110.955 121.046) (width 0.254) (layer F.Cu) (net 8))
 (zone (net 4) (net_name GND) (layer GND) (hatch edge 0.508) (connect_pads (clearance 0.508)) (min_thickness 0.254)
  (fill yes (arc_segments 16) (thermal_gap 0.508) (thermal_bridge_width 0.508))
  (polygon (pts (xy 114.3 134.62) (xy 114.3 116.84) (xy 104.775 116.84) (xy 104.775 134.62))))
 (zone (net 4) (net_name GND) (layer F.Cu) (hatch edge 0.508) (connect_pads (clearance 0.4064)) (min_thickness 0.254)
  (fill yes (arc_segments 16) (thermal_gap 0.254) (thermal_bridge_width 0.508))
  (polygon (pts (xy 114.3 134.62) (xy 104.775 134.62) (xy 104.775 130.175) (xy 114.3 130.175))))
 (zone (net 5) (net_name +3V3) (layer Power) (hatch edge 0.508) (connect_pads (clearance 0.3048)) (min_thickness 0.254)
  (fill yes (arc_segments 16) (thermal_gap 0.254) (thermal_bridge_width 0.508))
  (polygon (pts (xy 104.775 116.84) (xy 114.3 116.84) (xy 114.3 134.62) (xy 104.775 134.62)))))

